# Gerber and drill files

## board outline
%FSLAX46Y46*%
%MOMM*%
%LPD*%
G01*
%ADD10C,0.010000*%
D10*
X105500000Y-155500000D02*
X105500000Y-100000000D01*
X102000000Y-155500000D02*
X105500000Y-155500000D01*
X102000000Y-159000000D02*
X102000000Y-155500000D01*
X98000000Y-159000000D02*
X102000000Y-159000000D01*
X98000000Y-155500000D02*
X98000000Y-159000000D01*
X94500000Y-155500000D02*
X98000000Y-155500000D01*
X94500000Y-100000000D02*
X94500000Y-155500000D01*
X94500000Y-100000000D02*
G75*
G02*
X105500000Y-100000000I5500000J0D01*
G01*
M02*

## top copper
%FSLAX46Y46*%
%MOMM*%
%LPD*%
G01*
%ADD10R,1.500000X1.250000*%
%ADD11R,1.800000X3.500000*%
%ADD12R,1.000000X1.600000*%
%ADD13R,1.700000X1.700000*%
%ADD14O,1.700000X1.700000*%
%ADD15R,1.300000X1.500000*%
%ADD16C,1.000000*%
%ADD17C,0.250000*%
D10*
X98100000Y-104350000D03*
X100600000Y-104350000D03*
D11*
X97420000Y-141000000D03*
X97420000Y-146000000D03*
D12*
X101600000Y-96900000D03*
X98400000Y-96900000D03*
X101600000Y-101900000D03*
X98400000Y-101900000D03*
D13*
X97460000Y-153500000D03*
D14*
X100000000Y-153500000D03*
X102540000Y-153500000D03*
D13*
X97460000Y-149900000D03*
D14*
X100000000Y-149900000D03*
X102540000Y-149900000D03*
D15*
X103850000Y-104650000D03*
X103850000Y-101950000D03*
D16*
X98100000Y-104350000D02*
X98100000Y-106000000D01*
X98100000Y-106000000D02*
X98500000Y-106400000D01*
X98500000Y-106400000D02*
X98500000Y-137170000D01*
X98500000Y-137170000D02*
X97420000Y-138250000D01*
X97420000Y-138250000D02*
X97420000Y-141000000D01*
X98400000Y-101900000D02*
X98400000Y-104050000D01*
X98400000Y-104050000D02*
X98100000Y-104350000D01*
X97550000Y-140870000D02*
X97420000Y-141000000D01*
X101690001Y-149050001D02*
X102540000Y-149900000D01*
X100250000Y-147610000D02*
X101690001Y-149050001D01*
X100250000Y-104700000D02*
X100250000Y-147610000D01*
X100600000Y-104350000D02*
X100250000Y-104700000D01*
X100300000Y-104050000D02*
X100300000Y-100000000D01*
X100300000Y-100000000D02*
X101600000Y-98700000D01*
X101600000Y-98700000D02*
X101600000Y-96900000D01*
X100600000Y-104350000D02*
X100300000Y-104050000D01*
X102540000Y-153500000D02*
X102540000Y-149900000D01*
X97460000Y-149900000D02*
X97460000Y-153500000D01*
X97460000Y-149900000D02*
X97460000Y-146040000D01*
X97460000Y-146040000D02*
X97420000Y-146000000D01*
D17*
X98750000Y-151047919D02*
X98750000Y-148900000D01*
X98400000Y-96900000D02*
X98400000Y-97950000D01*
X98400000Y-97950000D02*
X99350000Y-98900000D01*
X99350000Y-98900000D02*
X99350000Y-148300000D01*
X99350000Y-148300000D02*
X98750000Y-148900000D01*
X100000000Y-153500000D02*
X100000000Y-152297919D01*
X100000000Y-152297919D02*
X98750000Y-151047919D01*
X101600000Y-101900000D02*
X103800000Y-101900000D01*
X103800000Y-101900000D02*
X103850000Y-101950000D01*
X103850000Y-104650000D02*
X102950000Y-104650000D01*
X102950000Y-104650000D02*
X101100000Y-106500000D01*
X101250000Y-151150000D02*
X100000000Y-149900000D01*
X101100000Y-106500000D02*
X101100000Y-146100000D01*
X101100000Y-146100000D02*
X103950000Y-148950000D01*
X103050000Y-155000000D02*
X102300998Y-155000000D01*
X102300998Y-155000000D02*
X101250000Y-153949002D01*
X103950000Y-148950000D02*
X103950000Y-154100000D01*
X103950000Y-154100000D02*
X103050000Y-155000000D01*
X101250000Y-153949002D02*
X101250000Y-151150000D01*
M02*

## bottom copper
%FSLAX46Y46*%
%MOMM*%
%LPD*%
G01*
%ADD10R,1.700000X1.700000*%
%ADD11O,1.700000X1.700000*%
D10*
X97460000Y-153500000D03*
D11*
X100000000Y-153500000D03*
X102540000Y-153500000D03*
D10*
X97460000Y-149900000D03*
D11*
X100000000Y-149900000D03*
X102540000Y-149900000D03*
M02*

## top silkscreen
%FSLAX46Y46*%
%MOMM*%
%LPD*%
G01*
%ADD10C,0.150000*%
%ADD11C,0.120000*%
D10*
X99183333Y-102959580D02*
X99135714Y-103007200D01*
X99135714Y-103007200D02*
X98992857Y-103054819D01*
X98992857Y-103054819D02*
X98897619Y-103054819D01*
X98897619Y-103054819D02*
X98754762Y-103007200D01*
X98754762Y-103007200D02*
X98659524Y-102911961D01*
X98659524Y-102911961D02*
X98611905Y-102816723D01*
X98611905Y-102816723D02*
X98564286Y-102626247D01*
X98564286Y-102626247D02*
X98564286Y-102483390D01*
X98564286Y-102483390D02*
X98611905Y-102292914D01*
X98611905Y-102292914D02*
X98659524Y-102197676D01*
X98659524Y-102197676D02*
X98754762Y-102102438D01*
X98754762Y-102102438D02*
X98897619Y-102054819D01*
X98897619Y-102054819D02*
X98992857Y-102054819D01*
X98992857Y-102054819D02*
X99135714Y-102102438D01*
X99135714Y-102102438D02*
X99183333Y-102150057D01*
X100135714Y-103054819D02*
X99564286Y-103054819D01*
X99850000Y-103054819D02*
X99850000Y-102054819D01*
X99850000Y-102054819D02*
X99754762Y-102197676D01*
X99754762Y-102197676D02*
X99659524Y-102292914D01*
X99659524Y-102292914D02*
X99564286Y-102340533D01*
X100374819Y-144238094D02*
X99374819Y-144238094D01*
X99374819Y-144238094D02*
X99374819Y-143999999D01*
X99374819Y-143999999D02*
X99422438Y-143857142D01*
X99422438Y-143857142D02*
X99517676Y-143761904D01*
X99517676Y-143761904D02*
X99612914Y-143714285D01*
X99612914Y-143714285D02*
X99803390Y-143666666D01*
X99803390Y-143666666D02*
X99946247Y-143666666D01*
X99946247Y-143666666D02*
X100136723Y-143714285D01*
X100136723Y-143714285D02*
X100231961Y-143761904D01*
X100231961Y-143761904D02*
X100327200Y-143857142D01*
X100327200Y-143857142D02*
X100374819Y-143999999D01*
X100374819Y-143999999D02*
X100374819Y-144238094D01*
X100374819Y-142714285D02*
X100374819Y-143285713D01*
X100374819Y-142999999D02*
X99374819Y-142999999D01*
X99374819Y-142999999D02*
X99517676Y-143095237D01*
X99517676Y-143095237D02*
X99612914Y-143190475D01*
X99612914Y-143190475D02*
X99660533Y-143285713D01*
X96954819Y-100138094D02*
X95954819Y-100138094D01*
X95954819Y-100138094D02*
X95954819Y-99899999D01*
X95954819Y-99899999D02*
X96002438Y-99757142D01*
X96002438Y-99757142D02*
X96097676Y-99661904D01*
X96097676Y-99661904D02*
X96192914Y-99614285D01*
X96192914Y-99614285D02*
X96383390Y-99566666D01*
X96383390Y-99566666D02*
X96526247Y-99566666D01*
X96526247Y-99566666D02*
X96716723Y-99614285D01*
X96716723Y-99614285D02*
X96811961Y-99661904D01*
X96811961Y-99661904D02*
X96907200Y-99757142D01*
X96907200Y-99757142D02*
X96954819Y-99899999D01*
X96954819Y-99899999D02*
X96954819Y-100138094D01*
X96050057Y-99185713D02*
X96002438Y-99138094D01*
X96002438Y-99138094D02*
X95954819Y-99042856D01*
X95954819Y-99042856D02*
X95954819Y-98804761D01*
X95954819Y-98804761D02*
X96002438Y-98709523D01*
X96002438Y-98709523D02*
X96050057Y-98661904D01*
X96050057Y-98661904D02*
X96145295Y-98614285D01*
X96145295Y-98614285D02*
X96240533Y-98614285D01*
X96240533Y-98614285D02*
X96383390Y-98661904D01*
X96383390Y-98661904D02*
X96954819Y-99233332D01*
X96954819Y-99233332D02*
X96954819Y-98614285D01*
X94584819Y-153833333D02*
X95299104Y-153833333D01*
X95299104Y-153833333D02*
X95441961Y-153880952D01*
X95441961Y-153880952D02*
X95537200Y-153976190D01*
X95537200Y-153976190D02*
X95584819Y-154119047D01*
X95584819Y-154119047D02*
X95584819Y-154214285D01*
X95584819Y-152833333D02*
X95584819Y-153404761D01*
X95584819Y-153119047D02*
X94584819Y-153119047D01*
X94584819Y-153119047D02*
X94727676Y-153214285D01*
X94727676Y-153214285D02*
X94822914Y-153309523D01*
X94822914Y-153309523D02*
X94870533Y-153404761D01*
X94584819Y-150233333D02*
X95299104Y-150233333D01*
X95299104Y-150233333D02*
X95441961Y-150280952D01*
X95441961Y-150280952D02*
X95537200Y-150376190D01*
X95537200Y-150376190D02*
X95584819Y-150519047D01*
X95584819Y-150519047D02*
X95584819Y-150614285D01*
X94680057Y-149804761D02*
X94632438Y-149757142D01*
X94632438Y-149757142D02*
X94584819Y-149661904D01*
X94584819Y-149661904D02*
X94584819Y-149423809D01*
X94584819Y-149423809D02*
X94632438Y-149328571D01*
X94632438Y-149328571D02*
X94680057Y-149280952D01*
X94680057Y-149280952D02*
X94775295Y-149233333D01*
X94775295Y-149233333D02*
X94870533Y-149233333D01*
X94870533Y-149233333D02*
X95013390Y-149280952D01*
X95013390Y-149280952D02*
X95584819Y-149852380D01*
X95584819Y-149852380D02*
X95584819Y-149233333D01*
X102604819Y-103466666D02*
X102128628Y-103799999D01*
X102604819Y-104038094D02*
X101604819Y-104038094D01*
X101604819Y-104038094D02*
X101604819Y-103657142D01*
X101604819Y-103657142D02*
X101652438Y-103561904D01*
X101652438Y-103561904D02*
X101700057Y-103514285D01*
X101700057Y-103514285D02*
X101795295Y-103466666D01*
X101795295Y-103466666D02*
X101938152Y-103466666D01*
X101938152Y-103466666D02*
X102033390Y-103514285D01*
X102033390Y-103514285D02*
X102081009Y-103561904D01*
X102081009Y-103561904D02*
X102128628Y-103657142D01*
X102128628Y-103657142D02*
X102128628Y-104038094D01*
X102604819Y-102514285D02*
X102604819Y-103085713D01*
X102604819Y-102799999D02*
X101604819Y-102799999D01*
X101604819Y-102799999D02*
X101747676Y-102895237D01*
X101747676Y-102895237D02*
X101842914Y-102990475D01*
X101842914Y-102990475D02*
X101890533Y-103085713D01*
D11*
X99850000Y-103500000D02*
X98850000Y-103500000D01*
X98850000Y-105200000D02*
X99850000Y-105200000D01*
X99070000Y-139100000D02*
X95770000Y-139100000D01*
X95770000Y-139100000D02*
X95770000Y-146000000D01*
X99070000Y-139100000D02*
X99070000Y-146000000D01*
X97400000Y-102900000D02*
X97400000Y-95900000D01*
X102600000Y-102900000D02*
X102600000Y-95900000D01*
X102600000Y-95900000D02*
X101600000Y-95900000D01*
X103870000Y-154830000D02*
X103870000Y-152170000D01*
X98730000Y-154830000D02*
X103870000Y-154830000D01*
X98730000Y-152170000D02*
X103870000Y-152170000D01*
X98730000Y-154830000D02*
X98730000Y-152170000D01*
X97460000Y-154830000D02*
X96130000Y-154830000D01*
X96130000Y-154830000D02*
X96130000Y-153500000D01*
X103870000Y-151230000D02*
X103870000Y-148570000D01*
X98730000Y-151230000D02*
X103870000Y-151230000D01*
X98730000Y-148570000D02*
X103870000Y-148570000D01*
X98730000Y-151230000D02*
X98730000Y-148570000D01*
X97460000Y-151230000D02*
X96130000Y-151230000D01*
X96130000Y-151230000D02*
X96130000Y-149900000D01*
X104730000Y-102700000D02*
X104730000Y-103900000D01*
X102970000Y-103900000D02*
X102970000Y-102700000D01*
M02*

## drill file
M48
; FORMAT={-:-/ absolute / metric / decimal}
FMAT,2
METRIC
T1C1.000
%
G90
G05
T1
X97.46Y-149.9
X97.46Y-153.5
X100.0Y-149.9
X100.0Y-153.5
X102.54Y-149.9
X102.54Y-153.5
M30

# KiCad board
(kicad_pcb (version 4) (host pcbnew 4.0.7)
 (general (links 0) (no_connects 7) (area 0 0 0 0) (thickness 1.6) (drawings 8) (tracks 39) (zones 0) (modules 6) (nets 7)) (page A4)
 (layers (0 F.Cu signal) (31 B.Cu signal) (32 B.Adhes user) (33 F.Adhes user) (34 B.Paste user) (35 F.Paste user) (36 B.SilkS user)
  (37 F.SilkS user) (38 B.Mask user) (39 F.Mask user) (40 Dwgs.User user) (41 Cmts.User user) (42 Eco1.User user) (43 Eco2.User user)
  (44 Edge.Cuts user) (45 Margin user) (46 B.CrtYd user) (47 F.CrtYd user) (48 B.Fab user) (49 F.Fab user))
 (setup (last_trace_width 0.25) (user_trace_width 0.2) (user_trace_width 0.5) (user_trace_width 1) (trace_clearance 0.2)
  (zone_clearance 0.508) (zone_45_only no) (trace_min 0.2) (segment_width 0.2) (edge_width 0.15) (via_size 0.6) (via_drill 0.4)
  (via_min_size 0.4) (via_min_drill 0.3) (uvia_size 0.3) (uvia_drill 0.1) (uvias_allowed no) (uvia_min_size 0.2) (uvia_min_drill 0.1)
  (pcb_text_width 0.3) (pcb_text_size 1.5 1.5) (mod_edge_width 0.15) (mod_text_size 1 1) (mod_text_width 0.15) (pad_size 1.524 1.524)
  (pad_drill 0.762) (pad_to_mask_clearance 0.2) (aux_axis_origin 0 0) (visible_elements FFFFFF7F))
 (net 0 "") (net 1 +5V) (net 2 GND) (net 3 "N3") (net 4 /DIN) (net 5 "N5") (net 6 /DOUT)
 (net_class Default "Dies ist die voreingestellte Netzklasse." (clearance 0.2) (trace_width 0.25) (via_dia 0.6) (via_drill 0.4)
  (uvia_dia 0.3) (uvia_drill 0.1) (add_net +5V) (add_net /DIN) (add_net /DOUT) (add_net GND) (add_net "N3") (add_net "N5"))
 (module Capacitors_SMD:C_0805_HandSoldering (layer F.Cu) (at 99.35 104.35)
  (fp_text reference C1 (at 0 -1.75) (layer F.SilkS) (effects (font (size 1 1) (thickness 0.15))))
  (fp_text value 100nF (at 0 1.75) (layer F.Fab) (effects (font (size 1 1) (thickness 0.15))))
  (fp_line (start 0.5 -0.85) (end -0.5 -0.85) (layer F.SilkS) (width 0.12))
  (fp_line (start -0.5 0.85) (end 0.5 0.85) (layer F.SilkS) (width 0.12))
  (pad 1 smd rect (at -1.25 0) (size 1.5 1.25) (layers F.Cu F.Paste F.Mask) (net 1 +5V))
  (pad 2 smd rect (at 1.25 0) (size 1.5 1.25) (layers F.Cu F.Paste F.Mask) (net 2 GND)))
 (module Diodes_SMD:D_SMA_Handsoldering (layer F.Cu) (at 97.42 143.5 270)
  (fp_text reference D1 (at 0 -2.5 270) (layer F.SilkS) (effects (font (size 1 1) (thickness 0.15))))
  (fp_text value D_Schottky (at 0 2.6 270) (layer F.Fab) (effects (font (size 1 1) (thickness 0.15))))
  (fp_line (start -4.4 -1.65) (end -4.4 1.65) (layer F.SilkS) (width 0.12))
  (fp_line (start -4.4 1.65) (end 2.5 1.65) (layer F.SilkS) (width 0.12))
  (fp_line (start -4.4 -1.65) (end 2.5 -1.65) (layer F.SilkS) (width 0.12))
  (pad 1 smd rect (at -2.5 0 270) (size 3.5 1.8) (layers F.Cu F.Paste F.Mask) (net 1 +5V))
  (pad 2 smd rect (at 2.5 0 270) (size 3.5 1.8) (layers F.Cu F.Paste F.Mask) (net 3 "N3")))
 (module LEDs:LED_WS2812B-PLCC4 (layer F.Cu) (at 100 99.4 90)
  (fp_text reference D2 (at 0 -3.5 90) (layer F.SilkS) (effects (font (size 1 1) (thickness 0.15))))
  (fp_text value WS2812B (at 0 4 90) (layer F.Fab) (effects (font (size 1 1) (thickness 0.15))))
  (fp_line (start -3.5 -2.6) (end 3.5 -2.6) (layer F.SilkS) (width 0.12))
  (fp_line (start -3.5 2.6) (end 3.5 2.6) (layer F.SilkS) (width 0.12))
  (fp_line (start 3.5 2.6) (end 3.5 1.6) (layer F.SilkS) (width 0.12))
  (pad 3 smd rect (at 2.5 1.6 90) (size 1.6 1) (layers F.Cu F.Paste F.Mask) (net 2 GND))
  (pad 4 smd rect (at 2.5 -1.6 90) (size 1.6 1) (layers F.Cu F.Paste F.Mask) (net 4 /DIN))
  (pad 2 smd rect (at -2.5 1.6 90) (size 1.6 1) (layers F.Cu F.Paste F.Mask) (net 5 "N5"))
  (pad 1 smd rect (at -2.5 -1.6 90) (size 1.6 1) (layers F.Cu F.Paste F.Mask) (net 1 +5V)))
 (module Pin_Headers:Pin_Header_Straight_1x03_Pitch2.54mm (layer F.Cu) (at 97.46 153.5 90)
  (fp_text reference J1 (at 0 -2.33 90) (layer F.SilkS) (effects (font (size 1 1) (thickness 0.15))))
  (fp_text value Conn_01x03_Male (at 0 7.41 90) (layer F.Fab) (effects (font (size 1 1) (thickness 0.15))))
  (fp_line (start -1.33 6.41) (end 1.33 6.41) (layer F.SilkS) (width 0.12))
  (fp_line (start -1.33 1.27) (end -1.33 6.41) (layer F.SilkS) (width 0.12))
  (fp_line (start 1.33 1.27) (end 1.33 6.41) (layer F.SilkS) (width 0.12))
  (fp_line (start -1.33 1.27) (end 1.33 1.27) (layer F.SilkS) (width 0.12))
  (fp_line (start -1.33 0) (end -1.33 -1.33) (layer F.SilkS) (width 0.12))
  (fp_line (start -1.33 -1.33) (end 0 -1.33) (layer F.SilkS) (width 0.12))
  (pad 1 thru_hole rect (at 0 0 90) (size 1.7 1.7) (drill 1) (layers *.Cu *.Mask) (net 3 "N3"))
  (pad 2 thru_hole oval (at 0 2.54 90) (size 1.7 1.7) (drill 1) (layers *.Cu *.Mask) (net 4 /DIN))
  (pad 3 thru_hole oval (at 0 5.08 90) (size 1.7 1.7) (drill 1) (layers *.Cu *.Mask) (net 2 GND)))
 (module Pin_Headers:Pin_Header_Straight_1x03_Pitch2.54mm (layer F.Cu) (at 97.46 149.9 90)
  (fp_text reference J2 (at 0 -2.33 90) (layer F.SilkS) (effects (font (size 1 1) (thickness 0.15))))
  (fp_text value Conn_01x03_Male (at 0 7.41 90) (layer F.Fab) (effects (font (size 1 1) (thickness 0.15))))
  (fp_line (start -1.33 6.41) (end 1.33 6.41) (layer F.SilkS) (width 0.12))
  (fp_line (start -1.33 1.27) (end -1.33 6.41) (layer F.SilkS) (width 0.12))
  (fp_line (start 1.33 1.27) (end 1.33 6.41) (layer F.SilkS) (width 0.12))
  (fp_line (start -1.33 1.27) (end 1.33 1.27) (layer F.SilkS) (width 0.12))
  (fp_line (start -1.33 0) (end -1.33 -1.33) (layer F.SilkS) (width 0.12))
  (fp_line (start -1.33 -1.33) (end 0 -1.33) (layer F.SilkS) (width 0.12))
  (pad 1 thru_hole rect (at 0 0 90) (size 1.7 1.7) (drill 1) (layers *.Cu *.Mask) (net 3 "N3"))
  (pad 2 thru_hole oval (at 0 2.54 90) (size 1.7 1.7) (drill 1) (layers *.Cu *.Mask) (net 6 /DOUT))
  (pad 3 thru_hole oval (at 0 5.08 90) (size 1.7 1.7) (drill 1) (layers *.Cu *.Mask) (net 2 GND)))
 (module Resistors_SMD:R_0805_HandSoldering (layer F.Cu) (at 103.85 103.3 90)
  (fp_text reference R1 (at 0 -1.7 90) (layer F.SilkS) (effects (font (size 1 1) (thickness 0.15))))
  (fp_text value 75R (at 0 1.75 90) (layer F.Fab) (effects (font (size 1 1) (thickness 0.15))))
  (fp_line (start 0.6 0.88) (end -0.6 0.88) (layer F.SilkS) (width 0.12))
  (fp_line (start -0.6 -0.88) (end 0.6 -0.88) (layer F.SilkS) (width 0.12))
  (pad 1 smd rect (at -1.35 0 90) (size 1.5 1.3) (layers F.Cu F.Paste F.Mask) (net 6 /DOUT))
  (pad 2 smd rect (at 1.35 0 90) (size 1.5 1.3) (layers F.Cu F.Paste F.Mask) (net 5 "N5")))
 (gr_line (start 105.5 155.5) (end 105.5 100) (layer Edge.Cuts) (width 0.01))
 (gr_line (start 102 155.5) (end 105.5 155.5) (layer Edge.Cuts) (width 0.01))
 (gr_line (start 102 159) (end 102 155.5) (layer Edge.Cuts) (width 0.01))
 (gr_line (start 98 159) (end 102 159) (layer Edge.Cuts) (width 0.01))
 (gr_line (start 98 155.5) (end 98 159) (layer Edge.Cuts) (width 0.01))
 (gr_line (start 94.5 155.5) (end 98 155.5) (layer Edge.Cuts) (width 0.01))
 (gr_line (start 94.5 100) (end 94.5 155.5) (layer Edge.Cuts) (width 0.01))
 (gr_arc (start 100 100) (end 94.5 100) (angle 180) (layer Edge.Cuts) (width 0.01))
 (segment (start 98.1 104.35) (end 98.1 106) (width 1) (layer F.Cu) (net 1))
 (segment (start 98.1 106) (end 98.5 106.4) (width 1) (layer F.Cu) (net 1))
 (segment (start 98.5 106.4) (end 98.5 137.17) (width 1) (layer F.Cu) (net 1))
 (segment (start 98.5 137.17) (end 97.42 138.25) (width 1) (layer F.Cu) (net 1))
 (segment (start 97.42 138.25) (end 97.42 141) (width 1) (layer F.Cu) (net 1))
 (segment (start 98.4 101.9) (end 98.4 104.05) (width 1) (layer F.Cu) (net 1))
 (segment (start 98.4 104.05) (end 98.1 104.35) (width 1) (layer F.Cu) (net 1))
 (segment (start 97.55 140.87) (end 97.42 141) (width 1) (layer F.Cu) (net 1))
 (segment (start 101.690001 149.050001) (end 102.54 149.9) (width 1) (layer F.Cu) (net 2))
 (segment (start 100.25 147.61) (end 101.690001 149.050001) (width 1) (layer F.Cu) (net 2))
 (segment (start 100.25 104.7) (end 100.25 147.61) (width 1) (layer F.Cu) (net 2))
 (segment (start 100.6 104.35) (end 100.25 104.7) (width 1) (layer F.Cu) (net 2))
 (segment (start 100.3 104.05) (end 100.3 100) (width 1) (layer F.Cu) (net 2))
 (segment (start 100.3 100) (end 101.6 98.7) (width 1) (layer F.Cu) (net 2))
 (segment (start 101.6 98.7) (end 101.6 96.9) (width 1) (layer F.Cu) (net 2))
 (segment (start 100.6 104.35) (end 100.3 104.05) (width 1) (layer F.Cu) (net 2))
 (segment (start 102.54 153.5) (end 102.54 149.9) (width 1) (layer F.Cu) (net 2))
 (segment (start 97.46 149.9) (end 97.46 153.5) (width 1) (layer F.Cu) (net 3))
 (segment (start 97.46 149.9) (end 97.46 146.04) (width 1) (layer F.Cu) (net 3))
 (segment (start 97.46 146.04) (end 97.42 146) (width 1) (layer F.Cu) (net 3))
 (segment (start 98.75 151.047919) (end 98.75 148.9) (width 0.25) (layer F.Cu) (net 4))
 (segment (start 98.4 96.9) (end 98.4 97.95) (width 0.25) (layer F.Cu) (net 4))
 (segment (start 98.4 97.95) (end 99.35 98.9) (width 0.25) (layer F.Cu) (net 4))
 (segment (start 99.35 98.9) (end 99.35 148.3) (width 0.25) (layer F.Cu) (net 4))
 (segment (start 99.35 148.3) (end 98.75 148.9) (width 0.25) (layer F.Cu) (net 4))
 (segment (start 100 153.5) (end 100 152.297919) (width 0.25) (layer F.Cu) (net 4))
 (segment (start 100 152.297919) (end 98.75 151.047919) (width 0.25) (layer F.Cu) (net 4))
 (segment (start 101.6 101.9) (end 103.8 101.9) (width 0.25) (layer F.Cu) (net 5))
 (segment (start 103.8 101.9) (end 103.85 101.95) (width 0.25) (layer F.Cu) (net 5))
 (segment (start 103.85 104.65) (end 102.95 104.65) (width 0.25) (layer F.Cu) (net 6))
 (segment (start 102.95 104.65) (end 101.1 106.5) (width 0.25) (layer F.Cu) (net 6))
 (segment (start 101.25 151.15) (end 100 149.9) (width 0.25) (layer F.Cu) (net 6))
 (segment (start 101.1 106.5) (end 101.1 146.1) (width 0.25) (layer F.Cu) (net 6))
 (segment (start 101.1 146.1) (end 103.95 148.95) (width 0.25) (layer F.Cu) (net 6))
 (segment (start 103.05 155) (end 102.300998 155) (width 0.25) (layer F.Cu) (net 6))
 (segment (start 102.300998 155) (end 101.25 153.949002) (width 0.25) (layer F.Cu) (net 6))
 (segment (start 103.95 148.95) (end 103.95 154.1) (width 0.25) (layer F.Cu) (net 6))
 (segment (start 103.95 154.1) (end 103.05 155) (width 0.25) (layer F.Cu) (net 6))
 (segment (start 101.25 153.949002) (end 101.25 151.15) (width 0.25) (layer F.Cu) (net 6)))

